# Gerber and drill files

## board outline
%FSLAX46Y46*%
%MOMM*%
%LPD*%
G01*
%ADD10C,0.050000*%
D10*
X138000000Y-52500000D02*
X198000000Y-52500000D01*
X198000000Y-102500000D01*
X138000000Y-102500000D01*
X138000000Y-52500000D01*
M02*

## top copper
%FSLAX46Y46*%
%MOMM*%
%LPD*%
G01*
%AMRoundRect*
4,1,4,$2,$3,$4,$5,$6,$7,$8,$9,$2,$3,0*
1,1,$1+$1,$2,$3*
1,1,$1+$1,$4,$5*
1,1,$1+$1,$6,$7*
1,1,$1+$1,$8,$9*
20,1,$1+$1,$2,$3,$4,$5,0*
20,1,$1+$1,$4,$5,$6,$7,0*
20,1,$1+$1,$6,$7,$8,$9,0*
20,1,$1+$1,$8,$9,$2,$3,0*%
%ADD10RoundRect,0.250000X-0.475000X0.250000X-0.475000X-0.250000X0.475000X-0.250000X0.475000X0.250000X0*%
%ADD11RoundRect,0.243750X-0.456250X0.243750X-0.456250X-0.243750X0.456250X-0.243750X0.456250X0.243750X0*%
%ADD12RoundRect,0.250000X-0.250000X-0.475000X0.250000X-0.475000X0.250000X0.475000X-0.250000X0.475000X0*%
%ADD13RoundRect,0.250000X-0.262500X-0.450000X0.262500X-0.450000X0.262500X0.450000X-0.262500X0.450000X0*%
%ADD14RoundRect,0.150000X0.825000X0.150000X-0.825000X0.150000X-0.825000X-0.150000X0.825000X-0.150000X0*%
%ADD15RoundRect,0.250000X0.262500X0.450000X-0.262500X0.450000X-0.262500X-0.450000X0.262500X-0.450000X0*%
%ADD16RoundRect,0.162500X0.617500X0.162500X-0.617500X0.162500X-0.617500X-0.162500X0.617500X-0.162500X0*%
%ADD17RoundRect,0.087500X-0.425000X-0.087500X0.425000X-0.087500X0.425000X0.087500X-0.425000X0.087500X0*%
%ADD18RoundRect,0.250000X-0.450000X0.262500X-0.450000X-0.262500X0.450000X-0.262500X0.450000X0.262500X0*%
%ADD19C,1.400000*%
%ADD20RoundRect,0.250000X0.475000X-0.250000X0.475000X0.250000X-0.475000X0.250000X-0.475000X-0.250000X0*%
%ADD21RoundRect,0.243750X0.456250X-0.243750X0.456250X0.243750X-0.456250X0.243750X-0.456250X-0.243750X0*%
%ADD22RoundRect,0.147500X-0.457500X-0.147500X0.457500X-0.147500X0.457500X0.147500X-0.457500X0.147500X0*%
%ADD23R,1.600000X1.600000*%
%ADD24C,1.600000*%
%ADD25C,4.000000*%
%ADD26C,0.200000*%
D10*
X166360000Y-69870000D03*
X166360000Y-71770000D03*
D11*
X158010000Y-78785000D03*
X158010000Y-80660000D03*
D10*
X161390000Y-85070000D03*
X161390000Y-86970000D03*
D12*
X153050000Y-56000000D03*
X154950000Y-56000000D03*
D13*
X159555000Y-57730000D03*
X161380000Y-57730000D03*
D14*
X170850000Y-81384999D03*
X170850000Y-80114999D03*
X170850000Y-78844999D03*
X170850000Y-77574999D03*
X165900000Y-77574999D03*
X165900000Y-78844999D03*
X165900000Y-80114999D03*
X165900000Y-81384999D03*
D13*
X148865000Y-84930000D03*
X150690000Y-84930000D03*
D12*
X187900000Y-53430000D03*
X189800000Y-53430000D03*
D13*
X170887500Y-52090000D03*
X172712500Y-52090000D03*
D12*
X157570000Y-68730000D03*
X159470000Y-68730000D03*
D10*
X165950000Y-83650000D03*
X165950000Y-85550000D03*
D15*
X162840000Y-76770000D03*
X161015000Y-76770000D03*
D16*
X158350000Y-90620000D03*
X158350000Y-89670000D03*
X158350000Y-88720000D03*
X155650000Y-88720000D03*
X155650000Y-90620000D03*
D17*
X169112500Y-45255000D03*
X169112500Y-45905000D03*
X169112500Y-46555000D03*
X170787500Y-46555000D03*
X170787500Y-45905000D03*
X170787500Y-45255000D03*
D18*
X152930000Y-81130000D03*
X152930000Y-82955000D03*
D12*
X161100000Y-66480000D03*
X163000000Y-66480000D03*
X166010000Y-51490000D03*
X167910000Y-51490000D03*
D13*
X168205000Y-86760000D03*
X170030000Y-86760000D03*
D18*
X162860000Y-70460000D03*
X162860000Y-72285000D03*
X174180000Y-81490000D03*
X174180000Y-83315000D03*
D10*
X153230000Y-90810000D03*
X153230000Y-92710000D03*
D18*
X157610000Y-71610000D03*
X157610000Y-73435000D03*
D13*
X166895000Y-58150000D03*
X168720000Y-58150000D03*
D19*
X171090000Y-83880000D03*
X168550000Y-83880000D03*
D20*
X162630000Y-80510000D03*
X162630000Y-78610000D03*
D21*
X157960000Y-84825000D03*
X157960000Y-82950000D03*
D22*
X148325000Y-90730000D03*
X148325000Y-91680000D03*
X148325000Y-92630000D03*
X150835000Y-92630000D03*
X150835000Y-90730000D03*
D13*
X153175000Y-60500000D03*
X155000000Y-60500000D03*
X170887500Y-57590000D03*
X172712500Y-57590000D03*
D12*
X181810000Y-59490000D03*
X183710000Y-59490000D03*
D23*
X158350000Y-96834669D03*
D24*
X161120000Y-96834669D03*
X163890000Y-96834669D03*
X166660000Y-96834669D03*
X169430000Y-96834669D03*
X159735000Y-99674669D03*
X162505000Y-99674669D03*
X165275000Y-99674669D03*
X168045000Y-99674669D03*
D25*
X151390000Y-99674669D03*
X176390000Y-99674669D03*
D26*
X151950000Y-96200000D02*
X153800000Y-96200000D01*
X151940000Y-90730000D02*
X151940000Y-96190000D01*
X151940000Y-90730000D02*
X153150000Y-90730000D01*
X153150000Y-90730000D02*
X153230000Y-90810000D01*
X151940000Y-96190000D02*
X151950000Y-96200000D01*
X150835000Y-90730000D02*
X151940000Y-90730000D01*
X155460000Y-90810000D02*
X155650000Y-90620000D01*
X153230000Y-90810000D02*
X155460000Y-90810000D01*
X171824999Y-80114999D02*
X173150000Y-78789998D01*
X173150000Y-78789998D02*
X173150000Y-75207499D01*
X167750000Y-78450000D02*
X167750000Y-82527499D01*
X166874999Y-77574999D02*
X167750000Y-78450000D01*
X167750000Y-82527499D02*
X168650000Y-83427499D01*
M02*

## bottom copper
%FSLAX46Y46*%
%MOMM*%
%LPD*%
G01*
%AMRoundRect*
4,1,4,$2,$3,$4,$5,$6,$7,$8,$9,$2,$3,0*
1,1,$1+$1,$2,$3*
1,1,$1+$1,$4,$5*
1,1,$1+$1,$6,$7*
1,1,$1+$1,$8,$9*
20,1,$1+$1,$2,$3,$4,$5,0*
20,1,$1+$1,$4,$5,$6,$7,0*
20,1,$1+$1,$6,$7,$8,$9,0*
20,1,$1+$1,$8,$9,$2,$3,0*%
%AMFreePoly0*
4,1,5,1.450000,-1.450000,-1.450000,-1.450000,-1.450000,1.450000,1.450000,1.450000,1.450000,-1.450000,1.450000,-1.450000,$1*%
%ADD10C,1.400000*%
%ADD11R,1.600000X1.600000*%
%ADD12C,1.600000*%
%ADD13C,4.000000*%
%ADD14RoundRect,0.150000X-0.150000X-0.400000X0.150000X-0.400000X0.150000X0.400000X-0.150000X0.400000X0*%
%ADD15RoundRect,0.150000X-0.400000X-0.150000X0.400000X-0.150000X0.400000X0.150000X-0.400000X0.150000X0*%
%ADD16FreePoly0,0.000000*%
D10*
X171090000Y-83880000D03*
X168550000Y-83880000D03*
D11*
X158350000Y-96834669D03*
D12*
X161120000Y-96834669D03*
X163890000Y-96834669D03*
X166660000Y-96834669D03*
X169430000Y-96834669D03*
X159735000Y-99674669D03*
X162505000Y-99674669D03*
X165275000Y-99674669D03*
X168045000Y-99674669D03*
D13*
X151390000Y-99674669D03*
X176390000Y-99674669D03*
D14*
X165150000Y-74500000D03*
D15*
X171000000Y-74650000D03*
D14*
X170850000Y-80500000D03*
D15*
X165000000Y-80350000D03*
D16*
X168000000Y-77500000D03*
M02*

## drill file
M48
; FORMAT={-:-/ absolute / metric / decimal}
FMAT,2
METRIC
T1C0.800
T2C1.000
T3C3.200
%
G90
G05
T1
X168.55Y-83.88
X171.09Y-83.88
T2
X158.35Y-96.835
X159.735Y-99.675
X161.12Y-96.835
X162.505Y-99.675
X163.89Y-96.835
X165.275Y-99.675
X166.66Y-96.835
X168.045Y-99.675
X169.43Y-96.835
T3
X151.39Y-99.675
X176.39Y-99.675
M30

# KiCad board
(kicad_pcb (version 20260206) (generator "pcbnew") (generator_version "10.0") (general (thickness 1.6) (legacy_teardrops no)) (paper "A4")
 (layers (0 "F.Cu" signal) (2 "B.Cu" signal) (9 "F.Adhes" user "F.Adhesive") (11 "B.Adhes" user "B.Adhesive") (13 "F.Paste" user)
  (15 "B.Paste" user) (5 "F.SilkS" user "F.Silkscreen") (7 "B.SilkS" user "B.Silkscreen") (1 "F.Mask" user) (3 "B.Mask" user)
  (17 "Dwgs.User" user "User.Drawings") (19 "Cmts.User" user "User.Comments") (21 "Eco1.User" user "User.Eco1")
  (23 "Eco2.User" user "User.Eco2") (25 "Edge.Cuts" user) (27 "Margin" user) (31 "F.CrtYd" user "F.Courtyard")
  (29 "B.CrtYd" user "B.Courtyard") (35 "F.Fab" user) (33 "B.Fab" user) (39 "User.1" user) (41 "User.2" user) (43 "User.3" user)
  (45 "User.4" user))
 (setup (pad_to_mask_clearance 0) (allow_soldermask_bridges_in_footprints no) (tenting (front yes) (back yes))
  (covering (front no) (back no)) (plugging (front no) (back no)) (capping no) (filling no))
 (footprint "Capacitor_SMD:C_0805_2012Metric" (layer "F.Cu") (at 166.36 70.82 -90)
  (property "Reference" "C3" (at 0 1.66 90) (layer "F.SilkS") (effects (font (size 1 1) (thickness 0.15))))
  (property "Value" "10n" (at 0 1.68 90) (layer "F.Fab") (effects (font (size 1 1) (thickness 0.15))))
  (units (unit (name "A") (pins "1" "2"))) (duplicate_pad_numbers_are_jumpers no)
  (pad "1" smd roundrect (at -0.95 0 270) (size 1 1.45) (layers "F.Cu" "F.Mask" "F.Paste") (roundrect_rratio 0.25) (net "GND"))
  (pad "2" smd roundrect (at 0.95 0 270) (size 1 1.45) (layers "F.Cu" "F.Mask" "F.Paste") (roundrect_rratio 0.25) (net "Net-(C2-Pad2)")))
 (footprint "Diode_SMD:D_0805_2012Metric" (layer "F.Cu") (at 158.01 79.7225 -90)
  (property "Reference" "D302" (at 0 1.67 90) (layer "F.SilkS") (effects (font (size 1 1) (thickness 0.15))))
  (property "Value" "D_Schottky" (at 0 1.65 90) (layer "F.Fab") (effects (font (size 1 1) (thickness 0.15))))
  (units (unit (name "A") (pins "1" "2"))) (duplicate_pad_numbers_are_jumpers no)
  (pad "1" smd roundrect (at -0.9375 0 270) (size 0.975 1.4) (layers "F.Cu" "F.Mask" "F.Paste") (roundrect_rratio 0.25) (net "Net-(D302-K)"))
  (pad "2" smd roundrect (at 0.9375 0 270) (size 0.975 1.4) (layers "F.Cu" "F.Mask" "F.Paste") (roundrect_rratio 0.25) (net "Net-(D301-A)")))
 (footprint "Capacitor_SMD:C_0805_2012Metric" (layer "F.Cu") (at 161.39 86.02 -90)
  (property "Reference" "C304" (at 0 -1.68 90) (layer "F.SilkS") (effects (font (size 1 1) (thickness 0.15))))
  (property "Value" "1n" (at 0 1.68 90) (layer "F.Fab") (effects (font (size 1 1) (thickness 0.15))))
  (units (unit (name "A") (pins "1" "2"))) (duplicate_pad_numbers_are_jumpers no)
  (pad "1" smd roundrect (at -0.95 0 270) (size 1 1.45) (layers "F.Cu" "F.Mask" "F.Paste") (roundrect_rratio 0.25) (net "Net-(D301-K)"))
  (pad "2" smd roundrect (at 0.95 0 270) (size 1 1.45) (layers "F.Cu" "F.Mask" "F.Paste") (roundrect_rratio 0.25) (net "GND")))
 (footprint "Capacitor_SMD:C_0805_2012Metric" (layer "F.Cu") (at 154 56)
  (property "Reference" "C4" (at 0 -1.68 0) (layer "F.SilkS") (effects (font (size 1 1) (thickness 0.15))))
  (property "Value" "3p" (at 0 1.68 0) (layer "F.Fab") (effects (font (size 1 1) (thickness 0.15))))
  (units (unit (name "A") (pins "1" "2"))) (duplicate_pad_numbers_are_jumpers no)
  (pad "1" smd roundrect (at -0.95 0) (size 1 1.45) (layers "F.Cu" "F.Mask" "F.Paste") (roundrect_rratio 0.25) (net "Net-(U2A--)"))
  (pad "2" smd roundrect (at 0.95 0) (size 1 1.45) (layers "F.Cu" "F.Mask" "F.Paste") (roundrect_rratio 0.25) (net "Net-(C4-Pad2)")))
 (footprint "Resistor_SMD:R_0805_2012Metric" (layer "F.Cu") (at 160.4675 57.73)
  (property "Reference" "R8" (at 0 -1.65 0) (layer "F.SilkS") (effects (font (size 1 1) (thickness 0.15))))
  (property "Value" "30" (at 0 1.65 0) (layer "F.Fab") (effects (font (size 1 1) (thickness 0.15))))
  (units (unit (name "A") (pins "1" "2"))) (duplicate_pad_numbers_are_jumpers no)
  (pad "1" smd roundrect (at -0.9125 0) (size 1.025 1.4) (layers "F.Cu" "F.Mask" "F.Paste") (roundrect_rratio 0.243902)
   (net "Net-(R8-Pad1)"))
  (pad "2" smd roundrect (at 0.9125 0) (size 1.025 1.4) (layers "F.Cu" "F.Mask" "F.Paste") (roundrect_rratio 0.243902)
   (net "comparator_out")))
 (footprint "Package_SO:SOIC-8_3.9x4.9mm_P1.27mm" (layer "F.Cu") (at 168.375 79.479999 180)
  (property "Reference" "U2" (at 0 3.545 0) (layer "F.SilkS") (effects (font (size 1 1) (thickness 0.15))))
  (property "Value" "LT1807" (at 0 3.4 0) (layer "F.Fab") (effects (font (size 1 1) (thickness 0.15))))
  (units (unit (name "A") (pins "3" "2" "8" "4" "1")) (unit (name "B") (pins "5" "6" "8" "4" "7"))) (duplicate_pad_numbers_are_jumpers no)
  (pad "1" smd roundrect (at -2.475 -1.905 180) (size 1.95 0.6) (layers "F.Cu" "F.Mask" "F.Paste") (roundrect_rratio 0.25)
   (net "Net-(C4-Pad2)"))
  (pad "2" smd roundrect (at -2.475 -0.635 180) (size 1.95 0.6) (layers "F.Cu" "F.Mask" "F.Paste") (roundrect_rratio 0.25)
   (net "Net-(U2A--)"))
  (pad "3" smd roundrect (at -2.475 0.635 180) (size 1.95 0.6) (layers "F.Cu" "F.Mask" "F.Paste") (roundrect_rratio 0.25) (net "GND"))
  (pad "4" smd roundrect (at -2.475 1.905 180) (size 1.95 0.6) (layers "F.Cu" "F.Mask" "F.Paste") (roundrect_rratio 0.25) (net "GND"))
  (pad "5" smd roundrect (at 2.475 1.905 180) (size 1.95 0.6) (layers "F.Cu" "F.Mask" "F.Paste") (roundrect_rratio 0.25)
   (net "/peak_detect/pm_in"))
  (pad "6" smd roundrect (at 2.475 0.635 180) (size 1.95 0.6) (layers "F.Cu" "F.Mask" "F.Paste") (roundrect_rratio 0.25)
   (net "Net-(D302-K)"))
  (pad "7" smd roundrect (at 2.475 -0.635 180) (size 1.95 0.6) (layers "F.Cu" "F.Mask" "F.Paste") (roundrect_rratio 0.25)
   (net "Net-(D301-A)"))
  (pad "8" smd roundrect (at 2.475 -1.905 180) (size 1.95 0.6) (layers "F.Cu" "F.Mask" "F.Paste") (roundrect_rratio 0.25) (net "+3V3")))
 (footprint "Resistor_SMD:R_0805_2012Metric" (layer "F.Cu") (at 149.7775 84.93)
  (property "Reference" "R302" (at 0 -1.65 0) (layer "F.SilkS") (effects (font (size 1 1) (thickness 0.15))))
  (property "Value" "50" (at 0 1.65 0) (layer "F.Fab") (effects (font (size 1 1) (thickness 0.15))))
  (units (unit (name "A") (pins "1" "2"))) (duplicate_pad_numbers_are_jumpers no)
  (pad "1" smd roundrect (at -0.9125 0) (size 1.025 1.4) (layers "F.Cu" "F.Mask" "F.Paste") (roundrect_rratio 0.243902) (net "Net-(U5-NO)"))
  (pad "2" smd roundrect (at 0.9125 0) (size 1.025 1.4) (layers "F.Cu" "F.Mask" "F.Paste") (roundrect_rratio 0.243902) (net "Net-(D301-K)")))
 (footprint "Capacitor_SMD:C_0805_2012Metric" (layer "F.Cu") (at 188.85 53.43)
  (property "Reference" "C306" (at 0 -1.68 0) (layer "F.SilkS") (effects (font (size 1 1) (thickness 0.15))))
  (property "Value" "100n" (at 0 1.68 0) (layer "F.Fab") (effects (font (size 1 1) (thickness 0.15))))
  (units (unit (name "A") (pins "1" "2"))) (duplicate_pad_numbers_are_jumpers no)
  (pad "1" smd roundrect (at -0.95 0) (size 1 1.45) (layers "F.Cu" "F.Mask" "F.Paste") (roundrect_rratio 0.25) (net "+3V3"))
  (pad "2" smd roundrect (at 0.95 0) (size 1 1.45) (layers "F.Cu" "F.Mask" "F.Paste") (roundrect_rratio 0.25) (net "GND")))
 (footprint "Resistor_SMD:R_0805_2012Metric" (layer "F.Cu") (at 171.8 52.09)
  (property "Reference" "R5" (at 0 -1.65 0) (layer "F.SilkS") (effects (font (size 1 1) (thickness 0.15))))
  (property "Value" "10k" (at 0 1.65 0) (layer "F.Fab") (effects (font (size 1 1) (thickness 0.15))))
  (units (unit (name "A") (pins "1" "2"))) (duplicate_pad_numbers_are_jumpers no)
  (pad "1" smd roundrect (at -0.9125 0) (size 1.025 1.4) (layers "F.Cu" "F.Mask" "F.Paste") (roundrect_rratio 0.243902) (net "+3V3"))
  (pad "2" smd roundrect (at 0.9125 0) (size 1.025 1.4) (layers "F.Cu" "F.Mask" "F.Paste") (roundrect_rratio 0.243902) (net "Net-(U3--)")))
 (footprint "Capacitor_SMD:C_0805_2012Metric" (layer "F.Cu") (at 158.52 68.73)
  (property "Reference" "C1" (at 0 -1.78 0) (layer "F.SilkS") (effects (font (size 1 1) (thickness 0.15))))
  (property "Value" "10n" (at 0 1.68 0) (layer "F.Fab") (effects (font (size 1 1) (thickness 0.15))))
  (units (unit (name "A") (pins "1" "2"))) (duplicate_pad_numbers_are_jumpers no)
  (pad "1" smd roundrect (at -0.95 0) (size 1 1.45) (layers "F.Cu" "F.Mask" "F.Paste") (roundrect_rratio 0.25) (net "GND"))
  (pad "2" smd roundrect (at 0.95 0) (size 1 1.45) (layers "F.Cu" "F.Mask" "F.Paste") (roundrect_rratio 0.25) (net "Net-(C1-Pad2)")))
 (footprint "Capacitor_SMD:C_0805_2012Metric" (layer "F.Cu") (at 165.95 84.6 -90)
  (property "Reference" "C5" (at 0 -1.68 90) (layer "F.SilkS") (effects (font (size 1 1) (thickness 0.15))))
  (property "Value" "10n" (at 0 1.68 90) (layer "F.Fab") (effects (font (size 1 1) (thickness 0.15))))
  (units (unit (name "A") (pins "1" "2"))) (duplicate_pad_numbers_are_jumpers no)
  (pad "1" smd roundrect (at -0.95 0 270) (size 1 1.45) (layers "F.Cu" "F.Mask" "F.Paste") (roundrect_rratio 0.25) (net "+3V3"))
  (pad "2" smd roundrect (at 0.95 0 270) (size 1 1.45) (layers "F.Cu" "F.Mask" "F.Paste") (roundrect_rratio 0.25) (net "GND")))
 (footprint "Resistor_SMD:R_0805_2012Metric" (layer "F.Cu") (at 161.9275 76.77 180)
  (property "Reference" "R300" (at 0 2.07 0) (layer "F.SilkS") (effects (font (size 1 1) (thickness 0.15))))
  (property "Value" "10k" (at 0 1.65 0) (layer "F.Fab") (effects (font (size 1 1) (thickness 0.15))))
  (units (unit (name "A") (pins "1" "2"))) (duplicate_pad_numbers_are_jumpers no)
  (pad "1" smd roundrect (at -0.9125 0 180) (size 1.025 1.4) (layers "F.Cu" "F.Mask" "F.Paste") (roundrect_rratio 0.243902)
   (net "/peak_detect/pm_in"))
  (pad "2" smd roundrect (at 0.9125 0 180) (size 1.025 1.4) (layers "F.Cu" "F.Mask" "F.Paste") (roundrect_rratio 0.243902) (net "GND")))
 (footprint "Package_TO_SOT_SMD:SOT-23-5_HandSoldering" (layer "F.Cu") (at 157 89.67 180)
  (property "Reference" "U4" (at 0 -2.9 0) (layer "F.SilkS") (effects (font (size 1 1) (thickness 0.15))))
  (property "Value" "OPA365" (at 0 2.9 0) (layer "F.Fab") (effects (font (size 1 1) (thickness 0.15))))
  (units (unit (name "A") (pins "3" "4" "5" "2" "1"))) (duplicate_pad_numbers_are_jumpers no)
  (pad "1" smd roundrect (at -1.35 -0.95 180) (size 1.56 0.65) (layers "F.Cu" "F.Mask" "F.Paste") (roundrect_rratio 0.25)
   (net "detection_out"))
  (pad "2" smd roundrect (at -1.35 0 180) (size 1.56 0.65) (layers "F.Cu" "F.Mask" "F.Paste") (roundrect_rratio 0.25) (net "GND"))
  (pad "3" smd roundrect (at -1.35 0.95 180) (size 1.56 0.65) (layers "F.Cu" "F.Mask" "F.Paste") (roundrect_rratio 0.25)
   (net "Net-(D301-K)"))
  (pad "4" smd roundrect (at 1.35 0.95 180) (size 1.56 0.65) (layers "F.Cu" "F.Mask" "F.Paste") (roundrect_rratio 0.25)
   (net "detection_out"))
  (pad "5" smd roundrect (at 1.35 -0.95 180) (size 1.56 0.65) (layers "F.Cu" "F.Mask" "F.Paste") (roundrect_rratio 0.25) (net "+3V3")))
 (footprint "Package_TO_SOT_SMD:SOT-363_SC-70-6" (layer "F.Cu") (at 169.95 45.905)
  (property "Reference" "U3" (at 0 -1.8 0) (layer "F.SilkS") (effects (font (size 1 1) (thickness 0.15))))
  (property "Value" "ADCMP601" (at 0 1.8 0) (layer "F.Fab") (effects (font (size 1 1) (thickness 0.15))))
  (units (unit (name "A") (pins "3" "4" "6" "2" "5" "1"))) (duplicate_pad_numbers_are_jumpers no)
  (pad "1" smd roundrect (at -0.8375 -0.65) (size 1.025 0.35) (layers "F.Cu" "F.Mask" "F.Paste") (roundrect_rratio 0.25)
   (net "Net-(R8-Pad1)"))
  (pad "2" smd roundrect (at -0.8375 0) (size 1.025 0.35) (layers "F.Cu" "F.Mask" "F.Paste") (roundrect_rratio 0.25) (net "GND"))
  (pad "3" smd roundrect (at -0.8375 0.65) (size 1.025 0.35) (layers "F.Cu" "F.Mask" "F.Paste") (roundrect_rratio 0.25)
   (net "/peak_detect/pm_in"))
  (pad "4" smd roundrect (at 0.8375 0.65) (size 1.025 0.35) (layers "F.Cu" "F.Mask" "F.Paste") (roundrect_rratio 0.25) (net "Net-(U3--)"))
  (pad "5" smd roundrect (at 0.8375 0) (size 1.025 0.35) (layers "F.Cu" "F.Mask" "F.Paste") (roundrect_rratio 0.25) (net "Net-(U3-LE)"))
  (pad "6" smd roundrect (at 0.8375 -0.65) (size 1.025 0.35) (layers "F.Cu" "F.Mask" "F.Paste") (roundrect_rratio 0.25) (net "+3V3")))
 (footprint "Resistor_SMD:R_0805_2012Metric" (layer "F.Cu") (at 152.93 82.0425 -90)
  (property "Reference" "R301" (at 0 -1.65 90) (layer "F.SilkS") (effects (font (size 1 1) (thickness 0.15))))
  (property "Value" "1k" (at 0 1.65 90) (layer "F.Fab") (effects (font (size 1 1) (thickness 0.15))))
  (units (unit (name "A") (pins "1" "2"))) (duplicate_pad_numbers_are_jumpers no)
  (pad "1" smd roundrect (at -0.9125 0 270) (size 1.025 1.4) (layers "F.Cu" "F.Mask" "F.Paste") (roundrect_rratio 0.243902)
   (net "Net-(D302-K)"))
  (pad "2" smd roundrect (at 0.9125 0 270) (size 1.025 1.4) (layers "F.Cu" "F.Mask" "F.Paste") (roundrect_rratio 0.243902)
   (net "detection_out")))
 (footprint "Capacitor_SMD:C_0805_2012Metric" (layer "F.Cu") (at 162.05 66.48)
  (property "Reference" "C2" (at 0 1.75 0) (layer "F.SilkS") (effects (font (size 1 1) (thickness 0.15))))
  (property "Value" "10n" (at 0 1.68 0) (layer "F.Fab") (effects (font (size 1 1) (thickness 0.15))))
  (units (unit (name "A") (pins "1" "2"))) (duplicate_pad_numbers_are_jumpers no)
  (pad "1" smd roundrect (at -0.95 0) (size 1 1.45) (layers "F.Cu" "F.Mask" "F.Paste") (roundrect_rratio 0.25) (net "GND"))
  (pad "2" smd roundrect (at 0.95 0) (size 1 1.45) (layers "F.Cu" "F.Mask" "F.Paste") (roundrect_rratio 0.25) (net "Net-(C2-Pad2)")))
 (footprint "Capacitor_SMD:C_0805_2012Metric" (layer "F.Cu") (at 166.96 51.49)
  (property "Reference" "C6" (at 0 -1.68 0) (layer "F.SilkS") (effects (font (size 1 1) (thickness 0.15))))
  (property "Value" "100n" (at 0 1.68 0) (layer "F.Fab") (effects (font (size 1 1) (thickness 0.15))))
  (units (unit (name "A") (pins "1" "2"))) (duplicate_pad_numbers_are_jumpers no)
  (pad "1" smd roundrect (at -0.95 0) (size 1 1.45) (layers "F.Cu" "F.Mask" "F.Paste") (roundrect_rratio 0.25) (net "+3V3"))
  (pad "2" smd roundrect (at 0.95 0) (size 1 1.45) (layers "F.Cu" "F.Mask" "F.Paste") (roundrect_rratio 0.25) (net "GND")))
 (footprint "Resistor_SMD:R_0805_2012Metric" (layer "F.Cu") (at 169.1175 86.76)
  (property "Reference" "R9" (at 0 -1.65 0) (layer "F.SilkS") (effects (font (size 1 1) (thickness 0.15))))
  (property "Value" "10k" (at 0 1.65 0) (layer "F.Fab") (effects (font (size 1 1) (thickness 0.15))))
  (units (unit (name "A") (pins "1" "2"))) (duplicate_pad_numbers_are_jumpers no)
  (pad "1" smd roundrect (at -0.9125 0) (size 1.025 1.4) (layers "F.Cu" "F.Mask" "F.Paste") (roundrect_rratio 0.243902)
   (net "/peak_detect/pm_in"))
  (pad "2" smd roundrect (at 0.9125 0) (size 1.025 1.4) (layers "F.Cu" "F.Mask" "F.Paste") (roundrect_rratio 0.243902) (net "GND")))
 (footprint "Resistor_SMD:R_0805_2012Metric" (layer "F.Cu") (at 162.86 71.3725 -90)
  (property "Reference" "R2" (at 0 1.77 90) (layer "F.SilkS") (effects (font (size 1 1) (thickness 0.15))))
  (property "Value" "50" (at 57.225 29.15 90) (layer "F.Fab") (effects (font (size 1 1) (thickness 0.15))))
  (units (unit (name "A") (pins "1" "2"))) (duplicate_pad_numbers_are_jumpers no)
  (pad "1" smd roundrect (at -0.9125 0 270) (size 1.025 1.4) (layers "F.Cu" "F.Mask" "F.Paste") (roundrect_rratio 0.243902)
   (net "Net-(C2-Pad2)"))
  (pad "2" smd roundrect (at 0.9125 0 270) (size 1.025 1.4) (layers "F.Cu" "F.Mask" "F.Paste") (roundrect_rratio 0.243902)
   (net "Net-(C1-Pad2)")))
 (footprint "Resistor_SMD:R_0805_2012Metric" (layer "F.Cu") (at 174.18 82.4025 -90)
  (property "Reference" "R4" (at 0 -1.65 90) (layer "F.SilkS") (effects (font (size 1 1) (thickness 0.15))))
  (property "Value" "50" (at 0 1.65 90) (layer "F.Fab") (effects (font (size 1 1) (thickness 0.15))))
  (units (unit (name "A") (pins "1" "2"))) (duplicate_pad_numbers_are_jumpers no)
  (pad "1" smd roundrect (at -0.9125 0 270) (size 1.025 1.4) (layers "F.Cu" "F.Mask" "F.Paste") (roundrect_rratio 0.243902)
   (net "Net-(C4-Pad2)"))
  (pad "2" smd roundrect (at 0.9125 0 270) (size 1.025 1.4) (layers "F.Cu" "F.Mask" "F.Paste") (roundrect_rratio 0.243902)
   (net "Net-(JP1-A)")))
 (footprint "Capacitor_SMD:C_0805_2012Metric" (layer "F.Cu") (at 153.23 91.76 -90)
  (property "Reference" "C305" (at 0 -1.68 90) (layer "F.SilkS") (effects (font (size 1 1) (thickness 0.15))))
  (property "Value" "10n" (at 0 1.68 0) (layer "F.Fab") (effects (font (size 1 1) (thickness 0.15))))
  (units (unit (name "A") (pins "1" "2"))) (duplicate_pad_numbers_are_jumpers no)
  (pad "1" smd roundrect (at -0.95 0 270) (size 1 1.45) (layers "F.Cu" "F.Mask" "F.Paste") (roundrect_rratio 0.25) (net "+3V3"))
  (pad "2" smd roundrect (at 0.95 0 270) (size 1 1.45) (layers "F.Cu" "F.Mask" "F.Paste") (roundrect_rratio 0.25) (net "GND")))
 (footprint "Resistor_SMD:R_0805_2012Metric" (layer "F.Cu") (at 157.61 72.5225 -90)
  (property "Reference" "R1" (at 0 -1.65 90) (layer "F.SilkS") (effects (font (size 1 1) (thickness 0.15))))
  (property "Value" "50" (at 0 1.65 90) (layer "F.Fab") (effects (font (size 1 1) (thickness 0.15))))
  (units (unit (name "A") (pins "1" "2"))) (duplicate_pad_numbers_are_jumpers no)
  (pad "1" smd roundrect (at -0.9125 0 270) (size 1.025 1.4) (layers "F.Cu" "F.Mask" "F.Paste") (roundrect_rratio 0.243902)
   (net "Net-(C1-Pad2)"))
  (pad "2" smd roundrect (at 0.9125 0 270) (size 1.025 1.4) (layers "F.Cu" "F.Mask" "F.Paste") (roundrect_rratio 0.243902) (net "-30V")))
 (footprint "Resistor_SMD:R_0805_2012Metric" (layer "F.Cu") (at 167.8075 58.15)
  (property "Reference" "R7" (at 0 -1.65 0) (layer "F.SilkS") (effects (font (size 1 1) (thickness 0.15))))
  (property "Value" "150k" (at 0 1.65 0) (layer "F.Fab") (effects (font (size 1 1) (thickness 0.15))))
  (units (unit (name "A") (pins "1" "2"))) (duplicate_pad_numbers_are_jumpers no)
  (pad "1" smd roundrect (at -0.9125 0) (size 1.025 1.4) (layers "F.Cu" "F.Mask" "F.Paste") (roundrect_rratio 0.243902) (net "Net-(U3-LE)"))
  (pad "2" smd roundrect (at 0.9125 0) (size 1.025 1.4) (layers "F.Cu" "F.Mask" "F.Paste") (roundrect_rratio 0.243902) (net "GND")))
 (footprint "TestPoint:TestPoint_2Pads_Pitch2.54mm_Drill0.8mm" (layer "F.Cu") (at 171.09 83.88 180)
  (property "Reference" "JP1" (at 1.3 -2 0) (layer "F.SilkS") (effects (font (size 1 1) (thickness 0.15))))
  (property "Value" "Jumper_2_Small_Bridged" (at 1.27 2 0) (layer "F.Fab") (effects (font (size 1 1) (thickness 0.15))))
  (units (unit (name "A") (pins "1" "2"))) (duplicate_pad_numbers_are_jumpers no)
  (pad "1" thru_hole circle (at 0 0 180) (size 1.4 1.4) (drill 0.8) (layers "*.Cu" "*.Mask") (remove_unused_layers no) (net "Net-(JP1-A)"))
  (pad "2" thru_hole circle (at 2.54 0 180) (size 1.4 1.4) (drill 0.8) (layers "*.Cu" "*.Mask") (remove_unused_layers no)
   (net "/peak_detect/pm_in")))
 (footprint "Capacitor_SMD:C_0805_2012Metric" (layer "F.Cu") (at 162.63 79.56 90)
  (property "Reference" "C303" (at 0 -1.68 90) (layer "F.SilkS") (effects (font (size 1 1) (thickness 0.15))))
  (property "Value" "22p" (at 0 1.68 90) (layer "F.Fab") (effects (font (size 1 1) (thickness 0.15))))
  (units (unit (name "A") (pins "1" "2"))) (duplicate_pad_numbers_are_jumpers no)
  (pad "1" smd roundrect (at -0.95 0 90) (size 1 1.45) (layers "F.Cu" "F.Mask" "F.Paste") (roundrect_rratio 0.25) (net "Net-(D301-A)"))
  (pad "2" smd roundrect (at 0.95 0 90) (size 1 1.45) (layers "F.Cu" "F.Mask" "F.Paste") (roundrect_rratio 0.25) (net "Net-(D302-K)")))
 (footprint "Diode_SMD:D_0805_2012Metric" (layer "F.Cu") (at 157.96 83.8875 90)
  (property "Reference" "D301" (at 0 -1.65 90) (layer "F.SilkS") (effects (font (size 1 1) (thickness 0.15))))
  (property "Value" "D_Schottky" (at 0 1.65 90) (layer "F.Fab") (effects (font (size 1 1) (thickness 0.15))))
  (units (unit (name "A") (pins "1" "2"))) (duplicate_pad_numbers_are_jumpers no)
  (pad "1" smd roundrect (at -0.9375 0 90) (size 0.975 1.4) (layers "F.Cu" "F.Mask" "F.Paste") (roundrect_rratio 0.25) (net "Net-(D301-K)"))
  (pad "2" smd roundrect (at 0.9375 0 90) (size 0.975 1.4) (layers "F.Cu" "F.Mask" "F.Paste") (roundrect_rratio 0.25) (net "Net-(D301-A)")))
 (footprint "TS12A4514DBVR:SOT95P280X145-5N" (layer "F.Cu") (at 149.58 91.68)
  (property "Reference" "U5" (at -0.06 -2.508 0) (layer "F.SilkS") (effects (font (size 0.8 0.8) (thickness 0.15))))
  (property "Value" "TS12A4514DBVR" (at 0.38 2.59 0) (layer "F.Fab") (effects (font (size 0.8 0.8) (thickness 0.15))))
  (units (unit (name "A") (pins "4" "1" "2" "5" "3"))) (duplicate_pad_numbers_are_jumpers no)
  (pad "1" smd roundrect (at -1.255 -0.95) (size 1.21 0.59) (layers "F.Cu" "F.Mask" "F.Paste") (roundrect_rratio 0.25) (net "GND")
   (solder_mask_margin 0.102))
  (pad "2" smd roundrect (at -1.255 0) (size 1.21 0.59) (layers "F.Cu" "F.Mask" "F.Paste") (roundrect_rratio 0.25) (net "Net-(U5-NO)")
   (solder_mask_margin 0.102))
  (pad "3" smd roundrect (at -1.255 0.95) (size 1.21 0.59) (layers "F.Cu" "F.Mask" "F.Paste") (roundrect_rratio 0.25) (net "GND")
   (solder_mask_margin 0.102))
  (pad "4" smd roundrect (at 1.255 0.95) (size 1.21 0.59) (layers "F.Cu" "F.Mask" "F.Paste") (roundrect_rratio 0.25) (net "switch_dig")
   (solder_mask_margin 0.102))
  (pad "5" smd roundrect (at 1.255 -0.95) (size 1.21 0.59) (layers "F.Cu" "F.Mask" "F.Paste") (roundrect_rratio 0.25) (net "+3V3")
   (solder_mask_margin 0.102)))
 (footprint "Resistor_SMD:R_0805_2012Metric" (layer "F.Cu") (at 154.0875 60.5)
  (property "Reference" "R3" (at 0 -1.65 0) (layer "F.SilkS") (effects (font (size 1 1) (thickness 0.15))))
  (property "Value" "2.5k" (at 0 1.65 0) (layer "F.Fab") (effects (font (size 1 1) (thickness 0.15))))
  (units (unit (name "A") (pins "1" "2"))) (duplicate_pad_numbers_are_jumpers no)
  (pad "1" smd roundrect (at -0.9125 0) (size 1.025 1.4) (layers "F.Cu" "F.Mask" "F.Paste") (roundrect_rratio 0.243902) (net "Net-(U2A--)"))
  (pad "2" smd roundrect (at 0.9125 0) (size 1.025 1.4) (layers "F.Cu" "F.Mask" "F.Paste") (roundrect_rratio 0.243902) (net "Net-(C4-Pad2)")))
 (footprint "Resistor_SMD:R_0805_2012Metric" (layer "F.Cu") (at 171.8 57.59)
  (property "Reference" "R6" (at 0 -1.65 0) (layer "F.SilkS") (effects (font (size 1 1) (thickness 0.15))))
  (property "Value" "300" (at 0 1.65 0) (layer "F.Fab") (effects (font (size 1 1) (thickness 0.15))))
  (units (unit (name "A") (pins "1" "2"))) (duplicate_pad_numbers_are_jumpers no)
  (pad "1" smd roundrect (at -0.9125 0) (size 1.025 1.4) (layers "F.Cu" "F.Mask" "F.Paste") (roundrect_rratio 0.243902) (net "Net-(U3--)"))
  (pad "2" smd roundrect (at 0.9125 0) (size 1.025 1.4) (layers "F.Cu" "F.Mask" "F.Paste") (roundrect_rratio 0.243902) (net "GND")))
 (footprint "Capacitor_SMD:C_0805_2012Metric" (layer "F.Cu") (at 182.76 59.49)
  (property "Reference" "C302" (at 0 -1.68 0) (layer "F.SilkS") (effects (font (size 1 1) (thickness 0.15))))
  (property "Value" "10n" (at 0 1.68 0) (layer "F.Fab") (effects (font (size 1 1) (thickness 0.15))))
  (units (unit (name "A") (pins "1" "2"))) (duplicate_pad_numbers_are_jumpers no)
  (pad "1" smd roundrect (at -0.95 0) (size 1 1.45) (layers "F.Cu" "F.Mask" "F.Paste") (roundrect_rratio 0.25) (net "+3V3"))
  (pad "2" smd roundrect (at 0.95 0) (size 1 1.45) (layers "F.Cu" "F.Mask" "F.Paste") (roundrect_rratio 0.25) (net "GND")))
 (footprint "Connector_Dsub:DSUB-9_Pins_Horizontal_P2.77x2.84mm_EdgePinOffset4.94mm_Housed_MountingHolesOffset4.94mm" (layer "F.Cu")
  (at 158.35 96.834669)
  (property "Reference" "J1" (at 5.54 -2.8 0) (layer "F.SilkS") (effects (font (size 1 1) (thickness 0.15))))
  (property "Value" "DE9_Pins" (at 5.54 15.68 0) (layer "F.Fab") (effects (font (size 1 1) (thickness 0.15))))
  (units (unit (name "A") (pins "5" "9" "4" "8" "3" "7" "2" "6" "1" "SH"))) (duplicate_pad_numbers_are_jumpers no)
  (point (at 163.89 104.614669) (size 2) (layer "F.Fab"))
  (pad "1" thru_hole rect (at 0 0) (size 1.6 1.6) (drill 1) (layers "*.Cu" "*.Mask") (remove_unused_layers no) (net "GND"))
  (pad "2" thru_hole circle (at 2.77 0) (size 1.6 1.6) (drill 1) (layers "*.Cu" "*.Mask") (remove_unused_layers no) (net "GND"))
  (pad "3" thru_hole circle (at 5.54 0) (size 1.6 1.6) (drill 1) (layers "*.Cu" "*.Mask") (remove_unused_layers no) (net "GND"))
  (pad "4" thru_hole circle (at 8.31 0) (size 1.6 1.6) (drill 1) (layers "*.Cu" "*.Mask") (remove_unused_layers no) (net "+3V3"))
  (pad "5" thru_hole circle (at 11.08 0) (size 1.6 1.6) (drill 1) (layers "*.Cu" "*.Mask") (remove_unused_layers no) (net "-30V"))
  (pad "6" thru_hole circle (at 1.385 2.84) (size 1.6 1.6) (drill 1) (layers "*.Cu" "*.Mask") (remove_unused_layers no)
   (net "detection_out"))
  (pad "7" thru_hole circle (at 4.155 2.84) (size 1.6 1.6) (drill 1) (layers "*.Cu" "*.Mask") (remove_unused_layers no)
   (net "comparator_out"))
  (pad "8" thru_hole circle (at 6.925 2.84) (size 1.6 1.6) (drill 1) (layers "*.Cu" "*.Mask") (remove_unused_layers no) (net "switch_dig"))
  (pad "9" thru_hole circle (at 9.695 2.84) (size 1.6 1.6) (drill 1) (layers "*.Cu" "*.Mask") (remove_unused_layers no) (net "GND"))
  (pad "SH" thru_hole circle (at -6.96 2.84) (size 4 4) (drill 3.2) (layers "*.Cu" "*.Mask") (remove_unused_layers no) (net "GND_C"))
  (pad "SH" thru_hole circle (at 18.04 2.84) (size 4 4) (drill 3.2) (layers "*.Cu" "*.Mask") (remove_unused_layers no) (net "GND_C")))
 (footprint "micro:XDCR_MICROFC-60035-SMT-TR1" (layer "B.Cu") (at 168 77.5)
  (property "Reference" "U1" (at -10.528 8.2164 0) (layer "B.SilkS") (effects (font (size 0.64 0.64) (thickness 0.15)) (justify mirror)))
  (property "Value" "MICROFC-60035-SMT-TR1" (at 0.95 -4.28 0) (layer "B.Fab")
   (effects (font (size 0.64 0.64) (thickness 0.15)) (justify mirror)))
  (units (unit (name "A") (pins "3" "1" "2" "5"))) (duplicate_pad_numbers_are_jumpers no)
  (pad "1" smd roundrect (at -2.85 -3) (size 0.6 1.1) (layers "B.Cu" "B.Mask" "B.Paste") (roundrect_rratio 0.25) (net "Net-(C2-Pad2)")
   (solder_mask_margin 0.102))
  (pad "2" smd roundrect (at 3 -2.85) (size 1.1 0.6) (layers "B.Cu" "B.Mask" "B.Paste") (roundrect_rratio 0.25)
   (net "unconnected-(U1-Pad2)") (solder_mask_margin 0.102))
  (pad "3" smd roundrect (at 2.85 3) (size 0.6 1.1) (layers "B.Cu" "B.Mask" "B.Paste") (roundrect_rratio 0.25) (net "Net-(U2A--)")
   (solder_mask_margin 0.102))
  (pad "4" smd roundrect (at -3 2.85) (size 1.1 0.6) (layers "B.Cu" "B.Mask" "B.Paste") (roundrect_rratio 0.25) (solder_mask_margin 0.102))
  (pad "5" smd custom (at 0 0) (size 2.9 2.9) (layers "B.Cu") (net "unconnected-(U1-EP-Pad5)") (options (clearance outline) (anchor rect))
   (primitives)))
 (gr_rect (start 138 52.5) (end 198 102.5) (stroke (width 0.05) (type solid)) (fill no) (layer "Edge.Cuts"))
 (segment (start 151.95 96.2) (end 153.8 96.2) (width 0.2) (layer "F.Cu") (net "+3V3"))
 (segment (start 151.94 90.73) (end 151.94 96.19) (width 0.2) (layer "F.Cu") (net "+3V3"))
 (segment (start 151.94 90.73) (end 153.15 90.73) (width 0.2) (layer "F.Cu") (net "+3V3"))
 (segment (start 153.15 90.73) (end 153.23 90.81) (width 0.2) (layer "F.Cu") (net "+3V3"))
 (segment (start 151.94 96.19) (end 151.95 96.2) (width 0.2) (layer "F.Cu") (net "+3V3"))
 (segment (start 150.835 90.73) (end 151.94 90.73) (width 0.2) (layer "F.Cu") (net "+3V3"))
 (segment (start 155.46 90.81) (end 155.65 90.62) (width 0.2) (layer "F.Cu") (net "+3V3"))
 (segment (start 153.23 90.81) (end 155.46 90.81) (width 0.2) (layer "F.Cu") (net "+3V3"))
 (segment (start 171.824999 80.114999) (end 173.15 78.789998) (width 0.2) (layer "F.Cu") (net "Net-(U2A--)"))
 (segment (start 173.15 78.789998) (end 173.15 75.207499) (width 0.2) (layer "F.Cu") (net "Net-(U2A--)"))
 (segment (start 167.75 78.45) (end 167.75 82.527499) (width 0.2) (layer "F.Cu") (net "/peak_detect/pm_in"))
 (segment (start 166.874999 77.574999) (end 167.75 78.45) (width 0.2) (layer "F.Cu") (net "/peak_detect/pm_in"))
 (segment (start 167.75 82.527499) (end 168.65 83.427499) (width 0.2) (layer "F.Cu") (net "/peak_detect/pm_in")))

